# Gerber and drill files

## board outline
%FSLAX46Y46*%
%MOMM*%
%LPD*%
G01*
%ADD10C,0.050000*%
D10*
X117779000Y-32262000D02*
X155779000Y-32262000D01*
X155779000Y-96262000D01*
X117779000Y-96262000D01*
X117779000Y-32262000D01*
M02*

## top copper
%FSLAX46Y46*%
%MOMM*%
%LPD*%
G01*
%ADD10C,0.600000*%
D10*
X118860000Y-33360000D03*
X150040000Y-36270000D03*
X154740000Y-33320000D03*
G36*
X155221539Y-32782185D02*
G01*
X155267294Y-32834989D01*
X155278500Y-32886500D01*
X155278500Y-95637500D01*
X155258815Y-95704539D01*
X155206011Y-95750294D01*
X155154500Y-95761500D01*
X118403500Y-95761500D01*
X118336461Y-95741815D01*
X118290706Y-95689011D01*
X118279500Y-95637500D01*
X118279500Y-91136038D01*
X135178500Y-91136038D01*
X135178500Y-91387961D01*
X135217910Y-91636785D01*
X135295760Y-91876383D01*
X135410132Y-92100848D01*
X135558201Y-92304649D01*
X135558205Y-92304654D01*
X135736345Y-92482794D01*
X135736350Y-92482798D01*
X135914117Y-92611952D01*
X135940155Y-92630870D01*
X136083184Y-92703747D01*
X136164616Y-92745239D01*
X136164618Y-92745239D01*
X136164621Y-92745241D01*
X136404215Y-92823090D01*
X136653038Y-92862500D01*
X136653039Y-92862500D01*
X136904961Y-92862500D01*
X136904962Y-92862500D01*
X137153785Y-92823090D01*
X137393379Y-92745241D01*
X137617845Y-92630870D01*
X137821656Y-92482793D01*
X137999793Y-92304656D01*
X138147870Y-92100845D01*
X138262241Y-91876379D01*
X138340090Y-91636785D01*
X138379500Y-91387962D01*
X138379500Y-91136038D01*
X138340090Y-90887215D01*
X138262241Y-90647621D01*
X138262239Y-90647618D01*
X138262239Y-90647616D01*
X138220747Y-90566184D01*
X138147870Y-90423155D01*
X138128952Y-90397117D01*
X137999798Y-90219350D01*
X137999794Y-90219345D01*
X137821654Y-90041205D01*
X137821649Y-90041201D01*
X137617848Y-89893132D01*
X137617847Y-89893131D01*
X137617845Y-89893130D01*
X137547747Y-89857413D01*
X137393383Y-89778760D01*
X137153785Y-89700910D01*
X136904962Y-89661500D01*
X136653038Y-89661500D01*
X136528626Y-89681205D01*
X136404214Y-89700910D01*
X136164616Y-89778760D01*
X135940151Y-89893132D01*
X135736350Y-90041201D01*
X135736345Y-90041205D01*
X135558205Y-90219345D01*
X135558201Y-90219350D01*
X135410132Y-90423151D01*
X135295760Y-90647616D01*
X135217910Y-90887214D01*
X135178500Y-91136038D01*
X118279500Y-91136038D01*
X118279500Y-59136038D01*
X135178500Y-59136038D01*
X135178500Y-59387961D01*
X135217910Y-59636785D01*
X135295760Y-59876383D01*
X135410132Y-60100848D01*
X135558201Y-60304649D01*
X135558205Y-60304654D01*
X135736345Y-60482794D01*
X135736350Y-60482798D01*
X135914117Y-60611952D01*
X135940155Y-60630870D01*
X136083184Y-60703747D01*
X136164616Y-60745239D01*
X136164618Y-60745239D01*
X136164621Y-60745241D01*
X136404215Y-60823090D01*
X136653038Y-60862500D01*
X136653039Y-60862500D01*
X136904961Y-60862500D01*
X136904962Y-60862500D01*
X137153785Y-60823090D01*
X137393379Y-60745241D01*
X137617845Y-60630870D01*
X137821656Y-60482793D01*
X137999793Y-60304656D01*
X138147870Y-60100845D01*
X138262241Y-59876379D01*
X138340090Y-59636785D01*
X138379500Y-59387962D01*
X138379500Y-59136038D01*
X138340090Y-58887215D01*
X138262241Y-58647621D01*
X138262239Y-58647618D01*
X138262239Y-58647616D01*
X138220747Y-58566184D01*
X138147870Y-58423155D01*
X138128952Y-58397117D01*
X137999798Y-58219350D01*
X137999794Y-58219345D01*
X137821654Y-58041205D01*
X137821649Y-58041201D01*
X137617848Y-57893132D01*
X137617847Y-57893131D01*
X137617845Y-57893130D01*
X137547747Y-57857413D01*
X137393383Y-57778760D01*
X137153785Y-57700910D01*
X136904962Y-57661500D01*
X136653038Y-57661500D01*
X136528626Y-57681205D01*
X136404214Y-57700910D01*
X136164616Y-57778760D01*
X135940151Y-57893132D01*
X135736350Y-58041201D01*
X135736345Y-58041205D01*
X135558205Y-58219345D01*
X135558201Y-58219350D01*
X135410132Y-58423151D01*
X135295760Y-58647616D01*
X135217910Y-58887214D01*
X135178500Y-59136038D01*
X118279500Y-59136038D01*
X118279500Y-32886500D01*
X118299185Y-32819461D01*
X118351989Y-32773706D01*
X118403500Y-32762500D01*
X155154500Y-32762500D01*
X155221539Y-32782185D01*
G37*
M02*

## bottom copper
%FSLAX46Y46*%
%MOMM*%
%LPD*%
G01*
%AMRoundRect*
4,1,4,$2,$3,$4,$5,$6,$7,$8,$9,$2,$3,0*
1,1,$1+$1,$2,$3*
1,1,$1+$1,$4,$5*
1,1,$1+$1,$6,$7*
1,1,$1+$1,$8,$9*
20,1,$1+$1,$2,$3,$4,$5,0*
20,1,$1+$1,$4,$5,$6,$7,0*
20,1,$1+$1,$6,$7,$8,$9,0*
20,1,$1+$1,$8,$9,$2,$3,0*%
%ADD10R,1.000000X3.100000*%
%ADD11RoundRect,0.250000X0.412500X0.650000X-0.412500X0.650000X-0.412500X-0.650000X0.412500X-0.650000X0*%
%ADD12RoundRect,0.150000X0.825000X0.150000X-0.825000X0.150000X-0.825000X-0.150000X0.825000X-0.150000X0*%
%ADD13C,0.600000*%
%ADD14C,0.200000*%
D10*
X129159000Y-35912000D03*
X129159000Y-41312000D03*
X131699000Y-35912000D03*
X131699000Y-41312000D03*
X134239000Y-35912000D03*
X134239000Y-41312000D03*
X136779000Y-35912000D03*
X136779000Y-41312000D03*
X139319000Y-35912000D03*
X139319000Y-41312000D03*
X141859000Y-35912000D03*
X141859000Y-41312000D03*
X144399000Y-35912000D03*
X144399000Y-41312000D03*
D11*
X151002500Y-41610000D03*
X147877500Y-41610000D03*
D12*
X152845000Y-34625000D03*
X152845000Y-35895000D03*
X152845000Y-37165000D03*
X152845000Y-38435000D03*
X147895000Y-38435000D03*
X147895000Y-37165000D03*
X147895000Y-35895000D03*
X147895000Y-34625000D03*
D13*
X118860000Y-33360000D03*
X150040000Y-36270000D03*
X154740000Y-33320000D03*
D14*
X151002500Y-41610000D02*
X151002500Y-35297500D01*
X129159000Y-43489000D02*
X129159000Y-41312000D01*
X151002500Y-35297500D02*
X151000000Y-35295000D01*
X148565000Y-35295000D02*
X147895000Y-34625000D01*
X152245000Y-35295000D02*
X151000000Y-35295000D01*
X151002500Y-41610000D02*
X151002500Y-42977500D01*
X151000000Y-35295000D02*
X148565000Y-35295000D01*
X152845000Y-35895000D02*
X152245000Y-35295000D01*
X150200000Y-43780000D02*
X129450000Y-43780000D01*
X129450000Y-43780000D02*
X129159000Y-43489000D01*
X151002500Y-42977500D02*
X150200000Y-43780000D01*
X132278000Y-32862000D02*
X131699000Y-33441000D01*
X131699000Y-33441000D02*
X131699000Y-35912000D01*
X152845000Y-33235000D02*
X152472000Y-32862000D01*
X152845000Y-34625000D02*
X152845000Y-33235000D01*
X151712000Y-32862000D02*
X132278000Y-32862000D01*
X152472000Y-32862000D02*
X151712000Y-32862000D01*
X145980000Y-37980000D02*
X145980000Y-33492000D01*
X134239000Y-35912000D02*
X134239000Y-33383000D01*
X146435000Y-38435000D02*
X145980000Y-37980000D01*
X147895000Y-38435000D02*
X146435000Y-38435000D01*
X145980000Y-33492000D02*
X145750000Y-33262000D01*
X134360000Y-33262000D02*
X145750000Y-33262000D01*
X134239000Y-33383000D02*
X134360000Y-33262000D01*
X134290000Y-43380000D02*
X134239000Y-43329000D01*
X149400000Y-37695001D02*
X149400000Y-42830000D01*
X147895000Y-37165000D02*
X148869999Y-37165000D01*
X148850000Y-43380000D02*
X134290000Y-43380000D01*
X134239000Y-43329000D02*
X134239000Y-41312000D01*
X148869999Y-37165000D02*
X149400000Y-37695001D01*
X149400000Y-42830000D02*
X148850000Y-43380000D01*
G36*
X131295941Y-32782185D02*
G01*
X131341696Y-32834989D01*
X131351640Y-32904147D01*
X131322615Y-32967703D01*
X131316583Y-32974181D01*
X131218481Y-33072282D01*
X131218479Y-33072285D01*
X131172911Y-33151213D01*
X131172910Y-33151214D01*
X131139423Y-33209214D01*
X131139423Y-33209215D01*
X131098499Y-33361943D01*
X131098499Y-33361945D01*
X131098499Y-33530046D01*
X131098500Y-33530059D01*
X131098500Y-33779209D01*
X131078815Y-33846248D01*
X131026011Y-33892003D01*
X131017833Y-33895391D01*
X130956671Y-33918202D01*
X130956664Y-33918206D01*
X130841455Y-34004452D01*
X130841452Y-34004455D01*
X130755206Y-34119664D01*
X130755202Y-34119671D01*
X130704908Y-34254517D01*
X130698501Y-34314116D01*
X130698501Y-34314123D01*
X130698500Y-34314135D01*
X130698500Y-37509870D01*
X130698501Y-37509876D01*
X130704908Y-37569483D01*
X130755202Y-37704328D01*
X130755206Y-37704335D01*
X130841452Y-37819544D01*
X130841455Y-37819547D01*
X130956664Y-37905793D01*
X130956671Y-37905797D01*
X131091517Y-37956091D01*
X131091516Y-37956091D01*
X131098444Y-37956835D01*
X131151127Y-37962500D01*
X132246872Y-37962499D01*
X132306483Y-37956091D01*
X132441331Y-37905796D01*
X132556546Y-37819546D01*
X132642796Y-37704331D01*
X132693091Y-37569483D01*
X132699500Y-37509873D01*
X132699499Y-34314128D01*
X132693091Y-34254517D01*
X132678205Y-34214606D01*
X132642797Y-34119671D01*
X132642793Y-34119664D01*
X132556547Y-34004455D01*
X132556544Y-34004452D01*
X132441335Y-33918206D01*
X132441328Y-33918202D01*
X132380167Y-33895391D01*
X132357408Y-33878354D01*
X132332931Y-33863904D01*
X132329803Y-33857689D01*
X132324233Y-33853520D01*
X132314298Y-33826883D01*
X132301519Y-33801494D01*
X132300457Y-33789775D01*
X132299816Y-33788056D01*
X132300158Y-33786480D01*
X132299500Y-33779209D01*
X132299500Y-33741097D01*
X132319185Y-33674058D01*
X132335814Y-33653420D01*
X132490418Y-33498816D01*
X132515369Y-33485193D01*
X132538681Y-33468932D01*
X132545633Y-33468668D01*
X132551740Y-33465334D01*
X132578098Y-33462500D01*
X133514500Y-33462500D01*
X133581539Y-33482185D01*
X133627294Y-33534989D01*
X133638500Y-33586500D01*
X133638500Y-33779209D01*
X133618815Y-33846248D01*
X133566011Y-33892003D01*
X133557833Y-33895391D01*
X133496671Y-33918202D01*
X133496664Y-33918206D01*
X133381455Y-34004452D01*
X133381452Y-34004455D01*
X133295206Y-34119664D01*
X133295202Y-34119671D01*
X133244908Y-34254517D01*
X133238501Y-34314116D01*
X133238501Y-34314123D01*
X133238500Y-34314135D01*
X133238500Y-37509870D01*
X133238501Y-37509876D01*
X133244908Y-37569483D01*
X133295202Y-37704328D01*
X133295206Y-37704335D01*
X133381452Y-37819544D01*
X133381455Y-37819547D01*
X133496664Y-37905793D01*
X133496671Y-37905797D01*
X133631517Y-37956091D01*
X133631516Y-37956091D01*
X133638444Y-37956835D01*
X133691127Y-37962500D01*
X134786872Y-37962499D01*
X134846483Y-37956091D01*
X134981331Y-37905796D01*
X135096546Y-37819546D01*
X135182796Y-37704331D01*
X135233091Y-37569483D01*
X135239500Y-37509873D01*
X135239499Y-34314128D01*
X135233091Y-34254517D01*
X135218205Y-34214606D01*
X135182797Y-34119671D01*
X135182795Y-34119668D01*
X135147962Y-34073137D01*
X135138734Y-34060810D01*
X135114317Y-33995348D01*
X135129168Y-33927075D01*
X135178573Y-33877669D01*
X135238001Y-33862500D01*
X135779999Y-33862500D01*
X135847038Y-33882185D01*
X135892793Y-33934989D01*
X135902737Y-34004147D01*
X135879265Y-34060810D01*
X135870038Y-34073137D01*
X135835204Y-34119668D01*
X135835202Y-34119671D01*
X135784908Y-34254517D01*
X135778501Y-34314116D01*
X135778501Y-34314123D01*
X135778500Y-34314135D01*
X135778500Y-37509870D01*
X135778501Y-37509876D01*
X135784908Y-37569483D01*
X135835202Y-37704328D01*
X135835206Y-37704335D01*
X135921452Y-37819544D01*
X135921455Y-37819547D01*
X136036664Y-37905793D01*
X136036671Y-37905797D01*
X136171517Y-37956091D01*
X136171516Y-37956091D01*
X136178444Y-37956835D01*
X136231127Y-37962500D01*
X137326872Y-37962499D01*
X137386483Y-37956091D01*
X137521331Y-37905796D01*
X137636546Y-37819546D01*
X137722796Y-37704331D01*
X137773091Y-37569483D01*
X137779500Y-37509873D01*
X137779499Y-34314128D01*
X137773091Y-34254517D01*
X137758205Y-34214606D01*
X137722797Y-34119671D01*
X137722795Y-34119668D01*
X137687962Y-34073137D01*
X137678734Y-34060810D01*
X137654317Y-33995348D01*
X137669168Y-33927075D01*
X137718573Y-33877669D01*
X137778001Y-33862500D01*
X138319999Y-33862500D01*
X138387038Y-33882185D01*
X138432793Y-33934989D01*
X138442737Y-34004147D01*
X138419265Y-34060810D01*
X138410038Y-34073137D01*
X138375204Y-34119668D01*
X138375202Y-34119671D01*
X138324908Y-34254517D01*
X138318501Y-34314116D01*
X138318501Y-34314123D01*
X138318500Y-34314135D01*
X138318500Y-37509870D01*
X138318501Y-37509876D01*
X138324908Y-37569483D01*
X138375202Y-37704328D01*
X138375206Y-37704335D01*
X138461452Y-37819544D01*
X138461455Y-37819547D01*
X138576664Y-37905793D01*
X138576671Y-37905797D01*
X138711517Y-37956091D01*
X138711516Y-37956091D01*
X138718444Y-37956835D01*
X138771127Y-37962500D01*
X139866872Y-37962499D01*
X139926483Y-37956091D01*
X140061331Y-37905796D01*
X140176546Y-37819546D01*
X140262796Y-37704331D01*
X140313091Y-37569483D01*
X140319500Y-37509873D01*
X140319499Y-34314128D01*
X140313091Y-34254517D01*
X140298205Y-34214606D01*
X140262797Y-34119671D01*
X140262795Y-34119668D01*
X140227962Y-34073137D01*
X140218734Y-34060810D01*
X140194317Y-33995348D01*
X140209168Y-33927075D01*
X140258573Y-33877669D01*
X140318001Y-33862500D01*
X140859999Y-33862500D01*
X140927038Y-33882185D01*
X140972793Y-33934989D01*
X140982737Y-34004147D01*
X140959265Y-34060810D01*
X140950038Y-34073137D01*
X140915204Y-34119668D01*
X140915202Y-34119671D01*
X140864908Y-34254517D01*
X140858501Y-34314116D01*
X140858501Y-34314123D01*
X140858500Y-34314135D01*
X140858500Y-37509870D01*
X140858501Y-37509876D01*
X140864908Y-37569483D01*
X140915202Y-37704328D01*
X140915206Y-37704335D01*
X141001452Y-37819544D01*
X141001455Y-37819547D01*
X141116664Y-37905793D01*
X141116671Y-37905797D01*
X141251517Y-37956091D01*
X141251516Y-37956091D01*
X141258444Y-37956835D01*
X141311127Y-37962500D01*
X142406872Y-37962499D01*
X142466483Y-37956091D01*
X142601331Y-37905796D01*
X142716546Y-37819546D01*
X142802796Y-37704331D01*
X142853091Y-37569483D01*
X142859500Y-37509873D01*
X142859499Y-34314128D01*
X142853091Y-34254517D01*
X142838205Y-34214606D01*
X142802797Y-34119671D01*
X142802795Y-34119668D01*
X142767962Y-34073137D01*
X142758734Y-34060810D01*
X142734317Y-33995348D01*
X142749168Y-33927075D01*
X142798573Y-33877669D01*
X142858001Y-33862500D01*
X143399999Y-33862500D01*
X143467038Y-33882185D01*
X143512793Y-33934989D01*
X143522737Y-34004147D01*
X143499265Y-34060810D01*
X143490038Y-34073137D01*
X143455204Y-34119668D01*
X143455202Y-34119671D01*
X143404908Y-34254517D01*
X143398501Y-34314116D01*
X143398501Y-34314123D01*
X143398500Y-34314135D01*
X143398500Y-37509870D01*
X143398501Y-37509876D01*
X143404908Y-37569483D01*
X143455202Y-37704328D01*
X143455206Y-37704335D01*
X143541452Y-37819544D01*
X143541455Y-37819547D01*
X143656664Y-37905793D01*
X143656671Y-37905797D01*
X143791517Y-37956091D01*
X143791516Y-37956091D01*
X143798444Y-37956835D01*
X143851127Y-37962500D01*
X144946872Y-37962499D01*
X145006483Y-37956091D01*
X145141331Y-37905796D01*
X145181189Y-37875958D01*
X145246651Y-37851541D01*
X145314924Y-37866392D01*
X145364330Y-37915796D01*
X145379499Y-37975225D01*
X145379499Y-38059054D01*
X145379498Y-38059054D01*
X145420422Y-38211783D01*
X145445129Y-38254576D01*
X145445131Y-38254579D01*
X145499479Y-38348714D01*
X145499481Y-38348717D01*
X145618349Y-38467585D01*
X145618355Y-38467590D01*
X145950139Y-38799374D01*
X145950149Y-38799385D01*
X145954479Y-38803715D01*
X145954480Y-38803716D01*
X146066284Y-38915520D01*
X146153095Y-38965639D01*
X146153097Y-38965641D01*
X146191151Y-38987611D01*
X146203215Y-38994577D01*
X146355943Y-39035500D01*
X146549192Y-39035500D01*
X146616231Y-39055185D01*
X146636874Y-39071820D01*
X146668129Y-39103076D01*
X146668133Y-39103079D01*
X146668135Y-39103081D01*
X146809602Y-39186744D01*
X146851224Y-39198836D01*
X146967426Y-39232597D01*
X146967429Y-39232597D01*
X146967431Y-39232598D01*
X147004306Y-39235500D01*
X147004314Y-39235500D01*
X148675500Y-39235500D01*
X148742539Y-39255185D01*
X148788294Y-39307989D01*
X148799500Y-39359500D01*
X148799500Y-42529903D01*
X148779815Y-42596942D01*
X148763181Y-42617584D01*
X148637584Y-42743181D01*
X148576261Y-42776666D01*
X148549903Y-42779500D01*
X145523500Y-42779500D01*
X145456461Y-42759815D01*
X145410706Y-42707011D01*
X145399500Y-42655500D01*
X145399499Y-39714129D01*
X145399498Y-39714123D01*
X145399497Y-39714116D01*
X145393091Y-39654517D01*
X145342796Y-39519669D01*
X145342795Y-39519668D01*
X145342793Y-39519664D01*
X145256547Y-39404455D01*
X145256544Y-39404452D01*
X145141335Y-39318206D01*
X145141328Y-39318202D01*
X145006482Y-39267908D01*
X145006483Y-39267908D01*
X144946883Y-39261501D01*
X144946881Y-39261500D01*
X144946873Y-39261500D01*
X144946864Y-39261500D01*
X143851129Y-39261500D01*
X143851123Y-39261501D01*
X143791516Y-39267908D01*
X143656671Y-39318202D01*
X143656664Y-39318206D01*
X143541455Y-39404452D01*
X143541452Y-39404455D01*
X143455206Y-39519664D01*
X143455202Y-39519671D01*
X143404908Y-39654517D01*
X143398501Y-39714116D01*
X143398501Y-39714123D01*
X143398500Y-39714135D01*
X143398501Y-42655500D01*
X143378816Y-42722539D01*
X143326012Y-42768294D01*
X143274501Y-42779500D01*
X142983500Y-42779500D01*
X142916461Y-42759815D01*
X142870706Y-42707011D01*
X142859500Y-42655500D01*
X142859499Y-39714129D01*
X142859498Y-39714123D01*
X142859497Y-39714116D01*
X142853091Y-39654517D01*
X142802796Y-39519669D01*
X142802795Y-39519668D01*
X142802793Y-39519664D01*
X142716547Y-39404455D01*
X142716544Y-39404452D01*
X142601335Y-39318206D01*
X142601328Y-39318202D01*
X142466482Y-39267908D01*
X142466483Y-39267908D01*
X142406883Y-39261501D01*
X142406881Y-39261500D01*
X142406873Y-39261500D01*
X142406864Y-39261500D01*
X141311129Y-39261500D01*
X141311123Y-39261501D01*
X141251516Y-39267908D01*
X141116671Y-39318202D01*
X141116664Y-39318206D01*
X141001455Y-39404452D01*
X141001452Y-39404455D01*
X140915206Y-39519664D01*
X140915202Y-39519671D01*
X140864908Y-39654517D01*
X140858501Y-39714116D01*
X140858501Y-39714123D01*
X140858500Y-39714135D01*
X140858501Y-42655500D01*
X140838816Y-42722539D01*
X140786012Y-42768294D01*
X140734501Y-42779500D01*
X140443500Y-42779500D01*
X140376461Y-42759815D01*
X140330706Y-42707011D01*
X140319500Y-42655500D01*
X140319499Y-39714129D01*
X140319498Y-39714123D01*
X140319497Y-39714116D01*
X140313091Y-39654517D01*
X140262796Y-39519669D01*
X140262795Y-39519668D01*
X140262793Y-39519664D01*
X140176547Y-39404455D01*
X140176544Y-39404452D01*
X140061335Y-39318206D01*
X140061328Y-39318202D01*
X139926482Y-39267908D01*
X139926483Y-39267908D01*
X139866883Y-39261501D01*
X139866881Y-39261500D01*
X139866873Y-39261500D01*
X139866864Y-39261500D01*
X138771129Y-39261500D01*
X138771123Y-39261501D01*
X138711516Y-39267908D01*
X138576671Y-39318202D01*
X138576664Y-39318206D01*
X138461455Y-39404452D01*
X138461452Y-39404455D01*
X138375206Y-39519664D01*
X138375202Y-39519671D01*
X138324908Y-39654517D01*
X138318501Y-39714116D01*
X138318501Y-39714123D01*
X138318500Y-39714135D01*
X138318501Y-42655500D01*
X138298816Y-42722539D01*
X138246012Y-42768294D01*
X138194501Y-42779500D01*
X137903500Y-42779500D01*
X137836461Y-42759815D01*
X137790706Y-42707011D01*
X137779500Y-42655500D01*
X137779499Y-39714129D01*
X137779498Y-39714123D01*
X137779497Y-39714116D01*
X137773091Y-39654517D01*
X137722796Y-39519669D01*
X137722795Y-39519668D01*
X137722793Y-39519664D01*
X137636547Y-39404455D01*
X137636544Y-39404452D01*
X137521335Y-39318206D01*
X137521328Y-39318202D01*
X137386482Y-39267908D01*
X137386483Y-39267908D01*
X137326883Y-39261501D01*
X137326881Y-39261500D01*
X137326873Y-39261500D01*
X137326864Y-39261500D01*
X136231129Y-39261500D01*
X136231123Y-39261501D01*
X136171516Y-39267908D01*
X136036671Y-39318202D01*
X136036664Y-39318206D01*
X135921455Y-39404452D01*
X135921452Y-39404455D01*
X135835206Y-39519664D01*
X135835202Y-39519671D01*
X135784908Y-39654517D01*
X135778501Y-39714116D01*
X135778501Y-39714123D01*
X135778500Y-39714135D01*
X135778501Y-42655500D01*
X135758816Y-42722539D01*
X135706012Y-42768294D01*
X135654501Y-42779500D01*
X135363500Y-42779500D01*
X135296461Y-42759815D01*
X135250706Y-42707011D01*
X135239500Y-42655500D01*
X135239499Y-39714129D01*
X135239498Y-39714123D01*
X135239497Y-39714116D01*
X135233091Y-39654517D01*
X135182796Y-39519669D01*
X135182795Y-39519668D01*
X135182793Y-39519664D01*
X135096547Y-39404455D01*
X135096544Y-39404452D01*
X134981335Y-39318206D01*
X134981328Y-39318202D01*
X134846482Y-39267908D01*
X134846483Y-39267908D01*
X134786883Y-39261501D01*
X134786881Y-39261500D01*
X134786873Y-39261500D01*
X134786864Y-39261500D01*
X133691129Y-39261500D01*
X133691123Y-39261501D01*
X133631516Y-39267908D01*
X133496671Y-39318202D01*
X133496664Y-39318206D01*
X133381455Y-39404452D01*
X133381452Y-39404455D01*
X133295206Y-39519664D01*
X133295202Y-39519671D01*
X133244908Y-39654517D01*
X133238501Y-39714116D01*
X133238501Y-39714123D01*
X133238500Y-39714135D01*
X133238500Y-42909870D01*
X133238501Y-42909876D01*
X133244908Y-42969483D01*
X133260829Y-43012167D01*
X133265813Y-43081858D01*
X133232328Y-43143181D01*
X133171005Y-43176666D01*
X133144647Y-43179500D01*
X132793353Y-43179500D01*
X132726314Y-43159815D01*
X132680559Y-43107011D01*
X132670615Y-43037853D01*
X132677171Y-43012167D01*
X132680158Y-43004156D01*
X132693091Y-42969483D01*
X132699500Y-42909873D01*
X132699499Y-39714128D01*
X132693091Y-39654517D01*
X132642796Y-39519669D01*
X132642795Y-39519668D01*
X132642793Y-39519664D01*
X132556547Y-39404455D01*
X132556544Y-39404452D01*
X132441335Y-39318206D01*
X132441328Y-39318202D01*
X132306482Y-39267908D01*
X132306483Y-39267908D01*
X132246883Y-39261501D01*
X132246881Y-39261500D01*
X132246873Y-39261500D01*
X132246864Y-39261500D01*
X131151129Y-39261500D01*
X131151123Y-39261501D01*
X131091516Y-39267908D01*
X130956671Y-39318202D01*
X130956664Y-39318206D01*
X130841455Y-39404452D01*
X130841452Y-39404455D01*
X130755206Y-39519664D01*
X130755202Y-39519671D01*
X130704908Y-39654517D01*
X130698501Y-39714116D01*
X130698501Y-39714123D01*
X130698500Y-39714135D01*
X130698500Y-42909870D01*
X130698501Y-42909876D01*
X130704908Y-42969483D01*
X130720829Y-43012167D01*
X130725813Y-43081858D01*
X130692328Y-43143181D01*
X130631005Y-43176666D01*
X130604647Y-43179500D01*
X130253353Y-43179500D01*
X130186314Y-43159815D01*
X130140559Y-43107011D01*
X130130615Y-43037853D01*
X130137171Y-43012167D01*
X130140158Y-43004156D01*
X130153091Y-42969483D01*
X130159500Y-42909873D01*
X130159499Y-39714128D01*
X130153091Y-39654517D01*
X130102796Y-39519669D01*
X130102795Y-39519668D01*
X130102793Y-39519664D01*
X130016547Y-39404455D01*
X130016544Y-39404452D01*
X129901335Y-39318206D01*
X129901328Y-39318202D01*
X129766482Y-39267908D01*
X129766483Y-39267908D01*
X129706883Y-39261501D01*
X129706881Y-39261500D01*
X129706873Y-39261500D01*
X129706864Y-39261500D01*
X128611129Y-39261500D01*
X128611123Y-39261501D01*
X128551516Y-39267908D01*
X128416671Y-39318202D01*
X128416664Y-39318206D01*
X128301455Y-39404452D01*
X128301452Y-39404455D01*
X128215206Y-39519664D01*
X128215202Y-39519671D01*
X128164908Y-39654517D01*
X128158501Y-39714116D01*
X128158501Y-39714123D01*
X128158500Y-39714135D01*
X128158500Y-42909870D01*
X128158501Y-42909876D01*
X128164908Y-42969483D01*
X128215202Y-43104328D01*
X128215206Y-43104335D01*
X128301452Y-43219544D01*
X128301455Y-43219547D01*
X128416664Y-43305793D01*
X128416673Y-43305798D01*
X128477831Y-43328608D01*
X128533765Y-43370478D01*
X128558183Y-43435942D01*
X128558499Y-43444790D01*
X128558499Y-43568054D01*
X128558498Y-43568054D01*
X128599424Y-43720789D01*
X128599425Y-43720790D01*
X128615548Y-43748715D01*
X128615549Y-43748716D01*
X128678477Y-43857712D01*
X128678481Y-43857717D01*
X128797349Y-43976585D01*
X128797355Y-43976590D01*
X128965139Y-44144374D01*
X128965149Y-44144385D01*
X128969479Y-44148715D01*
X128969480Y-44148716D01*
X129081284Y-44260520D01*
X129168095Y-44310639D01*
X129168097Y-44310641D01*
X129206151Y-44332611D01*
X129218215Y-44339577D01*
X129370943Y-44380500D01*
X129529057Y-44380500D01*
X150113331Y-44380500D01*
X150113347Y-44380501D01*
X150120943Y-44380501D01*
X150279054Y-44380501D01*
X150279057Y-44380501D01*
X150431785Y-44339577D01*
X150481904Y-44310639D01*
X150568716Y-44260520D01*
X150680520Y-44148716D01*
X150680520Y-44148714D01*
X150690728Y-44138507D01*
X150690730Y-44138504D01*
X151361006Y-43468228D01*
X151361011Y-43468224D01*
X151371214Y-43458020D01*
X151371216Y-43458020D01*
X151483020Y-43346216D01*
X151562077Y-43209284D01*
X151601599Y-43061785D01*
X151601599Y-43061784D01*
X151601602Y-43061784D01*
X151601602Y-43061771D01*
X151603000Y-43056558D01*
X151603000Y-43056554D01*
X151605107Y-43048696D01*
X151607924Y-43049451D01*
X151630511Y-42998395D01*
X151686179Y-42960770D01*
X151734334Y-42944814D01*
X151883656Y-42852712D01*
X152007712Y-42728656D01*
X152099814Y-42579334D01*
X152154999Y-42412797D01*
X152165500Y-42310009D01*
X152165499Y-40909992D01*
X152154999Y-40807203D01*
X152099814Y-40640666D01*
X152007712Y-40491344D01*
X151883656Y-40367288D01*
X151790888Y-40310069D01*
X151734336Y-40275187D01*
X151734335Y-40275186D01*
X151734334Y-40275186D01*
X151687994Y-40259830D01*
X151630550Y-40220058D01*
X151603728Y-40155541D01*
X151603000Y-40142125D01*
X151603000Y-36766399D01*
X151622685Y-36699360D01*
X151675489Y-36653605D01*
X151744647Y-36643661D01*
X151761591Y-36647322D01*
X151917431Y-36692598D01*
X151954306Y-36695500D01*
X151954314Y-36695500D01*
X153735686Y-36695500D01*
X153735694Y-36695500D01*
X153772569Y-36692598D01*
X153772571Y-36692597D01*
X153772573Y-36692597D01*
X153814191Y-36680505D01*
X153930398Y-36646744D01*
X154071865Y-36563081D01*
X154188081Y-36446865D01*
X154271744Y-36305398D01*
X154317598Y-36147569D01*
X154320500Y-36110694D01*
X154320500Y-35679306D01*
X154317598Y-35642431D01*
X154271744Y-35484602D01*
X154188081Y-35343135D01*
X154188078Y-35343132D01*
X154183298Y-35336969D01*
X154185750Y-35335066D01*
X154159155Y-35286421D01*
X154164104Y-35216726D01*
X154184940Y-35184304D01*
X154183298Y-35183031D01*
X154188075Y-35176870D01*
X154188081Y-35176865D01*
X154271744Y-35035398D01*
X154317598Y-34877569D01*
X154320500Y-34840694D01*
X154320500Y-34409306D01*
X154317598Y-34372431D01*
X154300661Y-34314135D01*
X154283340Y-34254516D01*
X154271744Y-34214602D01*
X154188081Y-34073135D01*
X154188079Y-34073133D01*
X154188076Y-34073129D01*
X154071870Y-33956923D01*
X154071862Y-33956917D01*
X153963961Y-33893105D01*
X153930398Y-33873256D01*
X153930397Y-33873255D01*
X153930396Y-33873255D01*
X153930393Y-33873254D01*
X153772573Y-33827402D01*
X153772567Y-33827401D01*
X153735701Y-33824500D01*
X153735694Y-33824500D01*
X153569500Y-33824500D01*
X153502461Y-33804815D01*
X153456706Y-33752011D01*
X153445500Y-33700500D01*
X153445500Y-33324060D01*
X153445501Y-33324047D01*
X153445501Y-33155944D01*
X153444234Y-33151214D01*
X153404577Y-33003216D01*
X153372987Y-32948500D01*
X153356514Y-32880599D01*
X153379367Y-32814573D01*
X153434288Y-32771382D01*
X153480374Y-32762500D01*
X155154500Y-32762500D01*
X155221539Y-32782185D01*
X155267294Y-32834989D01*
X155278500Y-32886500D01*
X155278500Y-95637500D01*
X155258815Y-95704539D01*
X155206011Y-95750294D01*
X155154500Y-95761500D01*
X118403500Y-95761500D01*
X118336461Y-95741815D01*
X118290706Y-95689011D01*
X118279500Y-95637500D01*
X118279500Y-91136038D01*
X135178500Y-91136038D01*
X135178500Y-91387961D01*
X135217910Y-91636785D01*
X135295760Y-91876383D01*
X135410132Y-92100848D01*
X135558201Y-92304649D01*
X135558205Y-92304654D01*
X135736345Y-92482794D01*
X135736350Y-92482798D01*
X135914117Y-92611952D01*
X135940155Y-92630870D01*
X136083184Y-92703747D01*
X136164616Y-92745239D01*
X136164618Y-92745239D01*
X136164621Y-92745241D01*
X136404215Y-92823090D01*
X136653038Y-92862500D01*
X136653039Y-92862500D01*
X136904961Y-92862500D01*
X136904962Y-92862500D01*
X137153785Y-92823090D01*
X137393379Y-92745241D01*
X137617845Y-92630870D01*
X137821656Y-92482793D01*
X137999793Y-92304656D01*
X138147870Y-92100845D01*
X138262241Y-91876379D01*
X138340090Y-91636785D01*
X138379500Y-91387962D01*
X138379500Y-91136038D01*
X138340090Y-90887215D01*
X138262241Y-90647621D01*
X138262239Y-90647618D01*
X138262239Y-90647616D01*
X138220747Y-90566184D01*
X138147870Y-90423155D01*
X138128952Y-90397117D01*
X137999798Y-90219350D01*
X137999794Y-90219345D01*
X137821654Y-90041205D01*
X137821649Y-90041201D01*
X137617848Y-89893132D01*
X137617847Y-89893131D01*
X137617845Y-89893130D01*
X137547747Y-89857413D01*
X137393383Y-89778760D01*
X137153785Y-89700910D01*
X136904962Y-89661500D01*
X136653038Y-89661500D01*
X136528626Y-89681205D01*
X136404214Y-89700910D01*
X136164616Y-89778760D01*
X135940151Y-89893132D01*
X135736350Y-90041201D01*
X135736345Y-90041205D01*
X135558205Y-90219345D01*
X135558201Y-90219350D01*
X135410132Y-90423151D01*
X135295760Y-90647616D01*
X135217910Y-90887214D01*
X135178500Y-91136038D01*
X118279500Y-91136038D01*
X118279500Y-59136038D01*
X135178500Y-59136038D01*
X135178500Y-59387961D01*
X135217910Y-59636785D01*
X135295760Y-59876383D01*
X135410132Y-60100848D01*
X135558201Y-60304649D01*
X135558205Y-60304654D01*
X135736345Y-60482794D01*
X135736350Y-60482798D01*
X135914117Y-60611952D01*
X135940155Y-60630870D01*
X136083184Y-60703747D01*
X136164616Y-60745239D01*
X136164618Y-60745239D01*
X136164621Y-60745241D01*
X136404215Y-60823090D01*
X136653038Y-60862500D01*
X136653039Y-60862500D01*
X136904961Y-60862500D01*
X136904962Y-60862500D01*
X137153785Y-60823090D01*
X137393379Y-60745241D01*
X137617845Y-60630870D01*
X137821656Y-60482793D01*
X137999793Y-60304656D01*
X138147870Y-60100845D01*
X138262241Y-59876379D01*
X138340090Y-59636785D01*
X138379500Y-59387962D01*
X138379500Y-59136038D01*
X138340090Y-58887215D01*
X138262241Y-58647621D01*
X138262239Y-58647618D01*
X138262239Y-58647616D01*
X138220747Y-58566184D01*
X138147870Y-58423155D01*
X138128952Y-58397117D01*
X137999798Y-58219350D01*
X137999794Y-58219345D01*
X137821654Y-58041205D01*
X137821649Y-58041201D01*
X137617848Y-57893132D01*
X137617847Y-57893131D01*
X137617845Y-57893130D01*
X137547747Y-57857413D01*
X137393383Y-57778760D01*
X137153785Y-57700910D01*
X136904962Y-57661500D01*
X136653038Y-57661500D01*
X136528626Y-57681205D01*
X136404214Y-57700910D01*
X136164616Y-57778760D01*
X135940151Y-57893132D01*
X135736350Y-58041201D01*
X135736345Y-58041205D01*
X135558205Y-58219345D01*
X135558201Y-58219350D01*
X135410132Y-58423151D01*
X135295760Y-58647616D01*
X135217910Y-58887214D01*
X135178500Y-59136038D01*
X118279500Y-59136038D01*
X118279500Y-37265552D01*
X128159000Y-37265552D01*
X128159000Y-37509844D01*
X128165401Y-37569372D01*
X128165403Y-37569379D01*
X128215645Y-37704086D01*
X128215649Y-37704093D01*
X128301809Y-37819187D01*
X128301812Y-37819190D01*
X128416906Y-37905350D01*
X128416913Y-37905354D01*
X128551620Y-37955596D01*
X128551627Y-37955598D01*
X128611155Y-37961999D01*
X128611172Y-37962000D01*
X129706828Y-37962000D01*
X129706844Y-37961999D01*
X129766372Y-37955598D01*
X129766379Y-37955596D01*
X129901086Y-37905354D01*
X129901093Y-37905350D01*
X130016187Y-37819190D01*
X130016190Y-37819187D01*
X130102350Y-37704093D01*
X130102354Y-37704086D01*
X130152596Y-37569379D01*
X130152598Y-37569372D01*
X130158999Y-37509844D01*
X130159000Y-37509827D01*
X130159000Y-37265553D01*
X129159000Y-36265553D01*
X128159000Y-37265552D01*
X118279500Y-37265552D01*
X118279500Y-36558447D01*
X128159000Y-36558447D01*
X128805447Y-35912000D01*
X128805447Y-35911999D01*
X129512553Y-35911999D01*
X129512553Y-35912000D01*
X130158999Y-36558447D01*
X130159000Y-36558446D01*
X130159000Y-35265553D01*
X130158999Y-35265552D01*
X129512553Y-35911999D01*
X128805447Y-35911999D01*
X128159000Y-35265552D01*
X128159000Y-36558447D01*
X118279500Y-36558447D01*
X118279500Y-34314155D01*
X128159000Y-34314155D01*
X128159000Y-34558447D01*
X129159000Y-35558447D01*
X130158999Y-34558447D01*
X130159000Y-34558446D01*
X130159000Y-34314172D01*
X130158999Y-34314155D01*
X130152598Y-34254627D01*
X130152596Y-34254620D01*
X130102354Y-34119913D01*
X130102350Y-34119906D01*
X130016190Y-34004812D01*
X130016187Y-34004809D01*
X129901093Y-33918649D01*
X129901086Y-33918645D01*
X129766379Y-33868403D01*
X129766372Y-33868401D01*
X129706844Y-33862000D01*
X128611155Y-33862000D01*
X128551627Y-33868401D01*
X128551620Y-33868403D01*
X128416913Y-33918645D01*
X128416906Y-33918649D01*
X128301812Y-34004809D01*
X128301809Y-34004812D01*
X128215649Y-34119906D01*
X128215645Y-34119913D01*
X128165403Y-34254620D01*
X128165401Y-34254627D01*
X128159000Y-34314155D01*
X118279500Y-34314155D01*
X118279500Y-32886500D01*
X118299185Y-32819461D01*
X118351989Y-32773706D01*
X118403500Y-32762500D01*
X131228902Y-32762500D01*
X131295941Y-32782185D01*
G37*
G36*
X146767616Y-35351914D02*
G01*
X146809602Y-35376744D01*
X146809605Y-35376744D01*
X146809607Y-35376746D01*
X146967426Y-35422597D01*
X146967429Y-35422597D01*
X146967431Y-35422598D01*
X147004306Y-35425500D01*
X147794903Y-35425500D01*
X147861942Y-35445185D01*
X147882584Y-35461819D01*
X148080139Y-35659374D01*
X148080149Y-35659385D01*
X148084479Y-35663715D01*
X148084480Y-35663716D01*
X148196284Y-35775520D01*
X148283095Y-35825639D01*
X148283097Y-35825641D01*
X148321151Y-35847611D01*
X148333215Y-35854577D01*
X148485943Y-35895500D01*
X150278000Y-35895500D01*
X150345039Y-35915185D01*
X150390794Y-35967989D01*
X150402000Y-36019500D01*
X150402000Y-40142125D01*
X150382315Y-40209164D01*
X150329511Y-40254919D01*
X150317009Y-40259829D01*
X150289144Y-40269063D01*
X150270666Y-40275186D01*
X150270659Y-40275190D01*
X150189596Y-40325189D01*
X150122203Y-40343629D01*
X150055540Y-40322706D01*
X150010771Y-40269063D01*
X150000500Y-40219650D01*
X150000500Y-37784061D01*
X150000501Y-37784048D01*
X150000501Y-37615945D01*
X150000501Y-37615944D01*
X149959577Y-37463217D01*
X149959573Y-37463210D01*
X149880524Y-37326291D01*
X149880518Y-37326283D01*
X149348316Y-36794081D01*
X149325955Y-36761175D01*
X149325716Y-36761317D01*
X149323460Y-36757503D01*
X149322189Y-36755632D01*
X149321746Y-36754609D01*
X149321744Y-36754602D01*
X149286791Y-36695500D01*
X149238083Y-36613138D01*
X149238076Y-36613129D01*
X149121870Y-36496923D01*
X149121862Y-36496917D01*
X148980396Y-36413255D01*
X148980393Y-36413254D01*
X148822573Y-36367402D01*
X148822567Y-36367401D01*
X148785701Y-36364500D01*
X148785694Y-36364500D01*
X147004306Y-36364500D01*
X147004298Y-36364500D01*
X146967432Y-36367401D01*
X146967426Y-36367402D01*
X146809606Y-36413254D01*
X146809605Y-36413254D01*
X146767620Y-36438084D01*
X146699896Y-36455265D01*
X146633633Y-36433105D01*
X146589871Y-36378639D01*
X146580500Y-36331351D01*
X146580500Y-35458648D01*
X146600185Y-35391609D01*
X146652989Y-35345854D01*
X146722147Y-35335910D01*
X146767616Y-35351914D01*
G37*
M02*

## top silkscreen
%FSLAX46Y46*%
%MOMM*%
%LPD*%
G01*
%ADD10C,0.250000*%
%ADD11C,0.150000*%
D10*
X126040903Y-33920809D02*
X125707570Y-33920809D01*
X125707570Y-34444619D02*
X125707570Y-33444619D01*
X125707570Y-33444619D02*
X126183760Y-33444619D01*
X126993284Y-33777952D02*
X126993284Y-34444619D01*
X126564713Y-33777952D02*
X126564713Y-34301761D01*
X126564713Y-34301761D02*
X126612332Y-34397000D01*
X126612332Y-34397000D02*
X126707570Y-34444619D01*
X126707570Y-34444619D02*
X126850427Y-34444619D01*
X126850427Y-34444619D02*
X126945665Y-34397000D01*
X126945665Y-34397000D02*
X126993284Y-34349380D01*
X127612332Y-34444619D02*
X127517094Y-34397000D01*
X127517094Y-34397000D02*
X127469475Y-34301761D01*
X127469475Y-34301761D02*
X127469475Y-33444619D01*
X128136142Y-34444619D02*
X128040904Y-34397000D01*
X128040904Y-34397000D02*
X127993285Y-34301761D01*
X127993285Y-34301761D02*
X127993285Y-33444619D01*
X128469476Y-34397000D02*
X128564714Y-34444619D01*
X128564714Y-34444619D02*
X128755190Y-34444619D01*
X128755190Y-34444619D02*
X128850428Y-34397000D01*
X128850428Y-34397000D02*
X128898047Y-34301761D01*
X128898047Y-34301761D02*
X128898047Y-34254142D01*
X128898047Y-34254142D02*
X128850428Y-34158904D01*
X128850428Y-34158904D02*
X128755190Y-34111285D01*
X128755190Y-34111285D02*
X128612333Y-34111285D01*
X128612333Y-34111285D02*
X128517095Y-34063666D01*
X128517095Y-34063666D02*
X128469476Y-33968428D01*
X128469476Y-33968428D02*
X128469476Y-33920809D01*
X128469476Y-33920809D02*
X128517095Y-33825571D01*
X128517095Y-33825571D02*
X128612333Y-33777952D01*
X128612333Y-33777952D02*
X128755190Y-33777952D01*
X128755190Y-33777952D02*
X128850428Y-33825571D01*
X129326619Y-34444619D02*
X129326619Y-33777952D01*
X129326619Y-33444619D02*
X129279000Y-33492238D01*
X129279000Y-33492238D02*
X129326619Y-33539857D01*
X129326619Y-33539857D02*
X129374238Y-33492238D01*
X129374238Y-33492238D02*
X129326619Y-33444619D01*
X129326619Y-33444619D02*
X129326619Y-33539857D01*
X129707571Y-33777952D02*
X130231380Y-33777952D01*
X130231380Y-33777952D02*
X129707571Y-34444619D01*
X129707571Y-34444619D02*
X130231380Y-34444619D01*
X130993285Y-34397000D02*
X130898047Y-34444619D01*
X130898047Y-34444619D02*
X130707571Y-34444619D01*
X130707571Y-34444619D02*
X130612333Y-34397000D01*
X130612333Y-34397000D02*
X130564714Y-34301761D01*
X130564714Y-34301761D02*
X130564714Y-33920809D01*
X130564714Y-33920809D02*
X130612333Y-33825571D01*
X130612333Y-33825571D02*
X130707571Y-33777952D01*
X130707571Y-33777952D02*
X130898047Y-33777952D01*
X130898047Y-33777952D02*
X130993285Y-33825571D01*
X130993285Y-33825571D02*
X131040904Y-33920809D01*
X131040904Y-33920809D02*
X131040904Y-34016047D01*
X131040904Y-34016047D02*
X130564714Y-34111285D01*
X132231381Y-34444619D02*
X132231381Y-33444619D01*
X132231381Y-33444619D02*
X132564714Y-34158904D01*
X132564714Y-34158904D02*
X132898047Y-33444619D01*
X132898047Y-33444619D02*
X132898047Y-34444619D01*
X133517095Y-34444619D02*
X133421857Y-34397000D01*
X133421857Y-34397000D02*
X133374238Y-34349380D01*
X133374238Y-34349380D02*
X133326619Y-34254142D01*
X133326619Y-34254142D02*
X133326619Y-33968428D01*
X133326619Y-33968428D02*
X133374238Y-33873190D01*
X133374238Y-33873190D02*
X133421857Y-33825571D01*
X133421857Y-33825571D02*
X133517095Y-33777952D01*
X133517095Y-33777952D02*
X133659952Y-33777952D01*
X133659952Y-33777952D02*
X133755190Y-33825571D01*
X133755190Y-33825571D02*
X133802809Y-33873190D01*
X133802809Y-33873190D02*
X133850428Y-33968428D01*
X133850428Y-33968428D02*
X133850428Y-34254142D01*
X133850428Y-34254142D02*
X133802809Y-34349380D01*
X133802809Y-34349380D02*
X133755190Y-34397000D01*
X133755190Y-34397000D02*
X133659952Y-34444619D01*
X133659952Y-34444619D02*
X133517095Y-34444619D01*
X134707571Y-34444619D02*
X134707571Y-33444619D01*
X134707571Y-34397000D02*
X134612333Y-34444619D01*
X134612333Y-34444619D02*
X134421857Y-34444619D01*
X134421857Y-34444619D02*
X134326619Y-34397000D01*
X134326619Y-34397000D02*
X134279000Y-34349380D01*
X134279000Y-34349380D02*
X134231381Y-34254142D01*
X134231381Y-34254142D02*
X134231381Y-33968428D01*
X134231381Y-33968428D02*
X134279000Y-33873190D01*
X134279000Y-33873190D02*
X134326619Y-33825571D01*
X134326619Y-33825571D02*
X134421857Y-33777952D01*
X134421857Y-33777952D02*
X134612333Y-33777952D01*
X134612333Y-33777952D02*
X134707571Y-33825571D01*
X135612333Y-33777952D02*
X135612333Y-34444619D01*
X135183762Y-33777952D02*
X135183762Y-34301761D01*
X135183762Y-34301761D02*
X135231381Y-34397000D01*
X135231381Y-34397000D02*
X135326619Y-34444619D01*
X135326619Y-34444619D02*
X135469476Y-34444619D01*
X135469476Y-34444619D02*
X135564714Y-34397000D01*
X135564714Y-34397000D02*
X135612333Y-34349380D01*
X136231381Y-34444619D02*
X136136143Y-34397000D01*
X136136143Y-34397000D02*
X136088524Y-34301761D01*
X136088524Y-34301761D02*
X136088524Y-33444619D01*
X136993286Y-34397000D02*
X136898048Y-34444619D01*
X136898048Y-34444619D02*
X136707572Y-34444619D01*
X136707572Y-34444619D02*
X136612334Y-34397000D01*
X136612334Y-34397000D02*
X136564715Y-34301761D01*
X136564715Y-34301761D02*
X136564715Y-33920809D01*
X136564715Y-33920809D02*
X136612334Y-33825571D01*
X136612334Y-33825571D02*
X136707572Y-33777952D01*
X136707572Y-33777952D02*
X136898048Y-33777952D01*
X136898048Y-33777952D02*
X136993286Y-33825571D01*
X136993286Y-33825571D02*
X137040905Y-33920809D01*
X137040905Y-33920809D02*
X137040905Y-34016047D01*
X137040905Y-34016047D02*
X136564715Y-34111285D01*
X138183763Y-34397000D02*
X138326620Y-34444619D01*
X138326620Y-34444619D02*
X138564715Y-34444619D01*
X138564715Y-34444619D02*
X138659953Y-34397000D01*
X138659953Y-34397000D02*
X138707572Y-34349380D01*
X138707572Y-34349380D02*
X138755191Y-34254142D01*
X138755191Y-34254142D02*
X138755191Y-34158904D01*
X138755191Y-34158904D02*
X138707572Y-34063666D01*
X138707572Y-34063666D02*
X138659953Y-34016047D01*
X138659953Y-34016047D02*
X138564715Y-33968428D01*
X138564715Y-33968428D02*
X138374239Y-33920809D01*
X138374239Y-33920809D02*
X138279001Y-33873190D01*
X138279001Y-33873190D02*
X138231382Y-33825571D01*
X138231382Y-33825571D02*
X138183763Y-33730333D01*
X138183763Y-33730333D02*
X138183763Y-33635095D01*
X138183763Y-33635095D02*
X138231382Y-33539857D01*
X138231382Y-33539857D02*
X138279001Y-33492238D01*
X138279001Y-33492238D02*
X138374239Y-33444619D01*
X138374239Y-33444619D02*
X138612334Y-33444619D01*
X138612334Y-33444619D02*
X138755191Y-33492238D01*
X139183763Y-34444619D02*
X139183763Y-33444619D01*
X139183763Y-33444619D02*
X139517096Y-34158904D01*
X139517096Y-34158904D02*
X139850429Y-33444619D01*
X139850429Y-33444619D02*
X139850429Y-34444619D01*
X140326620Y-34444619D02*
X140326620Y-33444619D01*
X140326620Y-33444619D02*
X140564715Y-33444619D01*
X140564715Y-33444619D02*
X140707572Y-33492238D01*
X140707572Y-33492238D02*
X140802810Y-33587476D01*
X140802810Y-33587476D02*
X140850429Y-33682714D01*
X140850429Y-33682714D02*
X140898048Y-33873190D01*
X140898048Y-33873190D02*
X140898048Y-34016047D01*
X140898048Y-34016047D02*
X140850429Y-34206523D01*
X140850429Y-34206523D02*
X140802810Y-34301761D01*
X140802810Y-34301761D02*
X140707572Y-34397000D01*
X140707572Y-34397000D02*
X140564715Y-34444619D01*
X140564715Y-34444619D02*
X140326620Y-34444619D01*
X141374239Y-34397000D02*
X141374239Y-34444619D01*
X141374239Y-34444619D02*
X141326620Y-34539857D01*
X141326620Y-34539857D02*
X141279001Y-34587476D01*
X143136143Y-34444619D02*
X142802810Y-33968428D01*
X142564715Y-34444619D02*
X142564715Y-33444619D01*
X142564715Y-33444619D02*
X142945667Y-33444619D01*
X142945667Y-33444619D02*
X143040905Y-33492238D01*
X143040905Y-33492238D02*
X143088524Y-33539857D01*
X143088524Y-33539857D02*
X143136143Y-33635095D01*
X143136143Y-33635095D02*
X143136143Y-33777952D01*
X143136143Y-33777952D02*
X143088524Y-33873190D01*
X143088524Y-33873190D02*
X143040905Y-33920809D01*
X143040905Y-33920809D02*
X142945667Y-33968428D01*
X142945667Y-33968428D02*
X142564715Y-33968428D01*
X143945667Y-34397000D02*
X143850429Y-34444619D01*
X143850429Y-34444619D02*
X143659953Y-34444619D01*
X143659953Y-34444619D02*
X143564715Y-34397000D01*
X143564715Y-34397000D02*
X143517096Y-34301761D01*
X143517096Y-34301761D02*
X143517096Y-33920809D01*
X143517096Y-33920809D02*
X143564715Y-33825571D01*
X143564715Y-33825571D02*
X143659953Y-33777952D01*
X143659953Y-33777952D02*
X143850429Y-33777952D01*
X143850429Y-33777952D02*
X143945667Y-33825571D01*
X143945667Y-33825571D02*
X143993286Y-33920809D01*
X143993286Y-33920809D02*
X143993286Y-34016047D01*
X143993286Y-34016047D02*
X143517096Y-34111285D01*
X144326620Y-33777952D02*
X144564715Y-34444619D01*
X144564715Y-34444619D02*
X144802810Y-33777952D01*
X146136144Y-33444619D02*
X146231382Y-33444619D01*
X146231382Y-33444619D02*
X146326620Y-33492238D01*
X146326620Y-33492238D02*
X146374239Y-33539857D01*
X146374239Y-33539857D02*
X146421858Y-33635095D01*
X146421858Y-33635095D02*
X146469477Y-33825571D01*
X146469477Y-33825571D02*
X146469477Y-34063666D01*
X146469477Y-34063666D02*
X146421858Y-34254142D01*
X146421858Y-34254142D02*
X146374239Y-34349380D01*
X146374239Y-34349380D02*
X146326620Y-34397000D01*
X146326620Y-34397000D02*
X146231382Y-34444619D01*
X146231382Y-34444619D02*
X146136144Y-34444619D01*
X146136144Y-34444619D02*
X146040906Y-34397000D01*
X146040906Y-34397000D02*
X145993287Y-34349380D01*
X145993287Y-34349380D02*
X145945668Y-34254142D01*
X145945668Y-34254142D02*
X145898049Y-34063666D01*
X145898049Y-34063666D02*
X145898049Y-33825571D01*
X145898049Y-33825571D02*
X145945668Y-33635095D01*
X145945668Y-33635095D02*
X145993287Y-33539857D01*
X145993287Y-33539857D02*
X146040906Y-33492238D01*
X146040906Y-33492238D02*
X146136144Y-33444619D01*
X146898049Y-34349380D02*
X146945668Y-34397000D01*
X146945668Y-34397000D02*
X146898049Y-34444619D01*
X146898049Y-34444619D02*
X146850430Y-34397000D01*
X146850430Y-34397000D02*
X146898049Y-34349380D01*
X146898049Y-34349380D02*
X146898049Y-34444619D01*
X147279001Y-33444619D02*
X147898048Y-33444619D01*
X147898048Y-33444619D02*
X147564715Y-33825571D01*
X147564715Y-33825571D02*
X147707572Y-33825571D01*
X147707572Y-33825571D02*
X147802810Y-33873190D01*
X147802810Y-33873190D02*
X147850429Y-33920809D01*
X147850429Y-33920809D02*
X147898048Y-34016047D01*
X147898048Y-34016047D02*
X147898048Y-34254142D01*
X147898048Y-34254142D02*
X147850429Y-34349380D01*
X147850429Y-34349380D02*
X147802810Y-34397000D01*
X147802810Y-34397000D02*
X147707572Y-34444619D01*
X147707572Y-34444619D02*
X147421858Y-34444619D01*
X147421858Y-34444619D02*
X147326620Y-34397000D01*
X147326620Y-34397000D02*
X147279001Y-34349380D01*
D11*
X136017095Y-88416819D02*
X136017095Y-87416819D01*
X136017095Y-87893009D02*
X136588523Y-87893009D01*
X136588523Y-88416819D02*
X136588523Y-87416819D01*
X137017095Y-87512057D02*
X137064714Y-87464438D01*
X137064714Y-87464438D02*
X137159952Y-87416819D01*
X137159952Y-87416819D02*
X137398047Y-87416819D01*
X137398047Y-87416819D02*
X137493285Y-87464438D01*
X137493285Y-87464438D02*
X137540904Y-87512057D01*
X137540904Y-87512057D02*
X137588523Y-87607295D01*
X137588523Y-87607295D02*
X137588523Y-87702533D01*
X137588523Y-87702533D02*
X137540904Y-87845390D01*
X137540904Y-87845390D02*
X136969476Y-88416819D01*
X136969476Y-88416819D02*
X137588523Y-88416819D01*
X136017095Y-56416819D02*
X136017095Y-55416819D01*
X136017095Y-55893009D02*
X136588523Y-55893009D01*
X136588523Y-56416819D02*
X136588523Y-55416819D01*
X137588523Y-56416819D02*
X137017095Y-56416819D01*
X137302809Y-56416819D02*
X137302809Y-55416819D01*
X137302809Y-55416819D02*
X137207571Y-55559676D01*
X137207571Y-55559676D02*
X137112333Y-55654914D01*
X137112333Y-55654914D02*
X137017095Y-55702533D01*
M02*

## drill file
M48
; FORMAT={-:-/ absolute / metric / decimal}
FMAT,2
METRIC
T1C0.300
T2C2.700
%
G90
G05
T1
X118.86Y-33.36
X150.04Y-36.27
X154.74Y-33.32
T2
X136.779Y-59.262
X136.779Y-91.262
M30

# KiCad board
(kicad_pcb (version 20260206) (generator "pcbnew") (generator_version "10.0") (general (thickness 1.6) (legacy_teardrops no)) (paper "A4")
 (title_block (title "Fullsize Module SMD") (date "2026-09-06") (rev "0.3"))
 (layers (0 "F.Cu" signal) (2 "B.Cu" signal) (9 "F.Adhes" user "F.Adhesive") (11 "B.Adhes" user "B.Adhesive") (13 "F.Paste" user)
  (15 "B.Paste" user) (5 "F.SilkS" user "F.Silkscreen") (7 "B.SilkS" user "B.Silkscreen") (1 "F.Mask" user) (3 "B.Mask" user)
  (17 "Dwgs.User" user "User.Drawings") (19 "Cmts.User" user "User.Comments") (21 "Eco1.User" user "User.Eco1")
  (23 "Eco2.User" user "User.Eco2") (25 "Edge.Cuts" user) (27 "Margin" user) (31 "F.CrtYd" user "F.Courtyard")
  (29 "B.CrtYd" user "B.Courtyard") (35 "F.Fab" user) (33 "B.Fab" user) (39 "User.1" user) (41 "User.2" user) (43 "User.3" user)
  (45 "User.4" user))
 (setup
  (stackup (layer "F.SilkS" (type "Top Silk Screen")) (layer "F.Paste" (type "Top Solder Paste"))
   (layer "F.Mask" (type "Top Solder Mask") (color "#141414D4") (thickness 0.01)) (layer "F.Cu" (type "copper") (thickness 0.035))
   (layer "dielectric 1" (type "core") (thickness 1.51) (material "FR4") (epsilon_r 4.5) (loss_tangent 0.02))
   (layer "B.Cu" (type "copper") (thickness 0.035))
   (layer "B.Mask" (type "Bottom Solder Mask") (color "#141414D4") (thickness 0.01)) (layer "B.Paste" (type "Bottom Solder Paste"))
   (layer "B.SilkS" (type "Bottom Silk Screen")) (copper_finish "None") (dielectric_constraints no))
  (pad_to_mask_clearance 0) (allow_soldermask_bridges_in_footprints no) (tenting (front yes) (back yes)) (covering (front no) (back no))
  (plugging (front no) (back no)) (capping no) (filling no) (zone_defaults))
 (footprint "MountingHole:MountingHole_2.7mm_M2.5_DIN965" (layer "F.Cu") (at 136.779 91.262)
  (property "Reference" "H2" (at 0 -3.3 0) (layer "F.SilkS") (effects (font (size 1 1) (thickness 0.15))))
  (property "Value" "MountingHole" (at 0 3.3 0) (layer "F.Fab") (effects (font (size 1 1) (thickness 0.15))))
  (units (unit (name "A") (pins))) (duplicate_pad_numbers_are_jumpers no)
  (pad "" np_thru_hole circle (at 0 0) (size 2.7 2.7) (drill 2.7) (layers "*.Cu" "*.Mask")))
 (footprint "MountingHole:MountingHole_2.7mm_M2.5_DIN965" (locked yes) (layer "F.Cu") (at 136.779 59.262)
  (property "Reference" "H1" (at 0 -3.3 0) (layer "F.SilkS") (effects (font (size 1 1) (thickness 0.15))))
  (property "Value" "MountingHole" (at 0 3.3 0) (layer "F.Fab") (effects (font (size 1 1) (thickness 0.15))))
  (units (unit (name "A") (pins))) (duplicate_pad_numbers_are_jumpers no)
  (pad "" np_thru_hole circle (at 0 0) (size 2.7 2.7) (drill 2.7) (layers "*.Cu" "*.Mask")))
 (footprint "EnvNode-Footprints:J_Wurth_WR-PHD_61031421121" (layer "B.Cu") (at 136.779 38.612 -90)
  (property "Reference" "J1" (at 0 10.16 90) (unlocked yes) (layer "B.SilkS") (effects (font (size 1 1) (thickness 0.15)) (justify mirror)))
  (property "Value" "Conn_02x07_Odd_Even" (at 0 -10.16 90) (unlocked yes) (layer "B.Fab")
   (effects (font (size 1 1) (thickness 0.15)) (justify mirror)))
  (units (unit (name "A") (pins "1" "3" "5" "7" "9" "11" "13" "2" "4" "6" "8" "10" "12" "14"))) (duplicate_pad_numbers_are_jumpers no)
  (pad "1" smd rect (at -2.7 7.62) (size 1 3.1) (layers "B.Cu" "B.Mask" "B.Paste") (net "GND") (thermal_bridge_angle 45))
  (pad "2" smd rect (at 2.7 7.62) (size 1 3.1) (layers "B.Cu" "B.Mask" "B.Paste") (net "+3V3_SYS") (thermal_bridge_angle 45))
  (pad "3" smd rect (at -2.7 5.08) (size 1 3.1) (layers "B.Cu" "B.Mask" "B.Paste") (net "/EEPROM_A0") (thermal_bridge_angle 45))
  (pad "4" smd rect (at 2.7 5.08) (size 1 3.1) (layers "B.Cu" "B.Mask" "B.Paste") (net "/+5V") (thermal_bridge_angle 45))
  (pad "5" smd rect (at -2.7 2.54) (size 1 3.1) (layers "B.Cu" "B.Mask" "B.Paste") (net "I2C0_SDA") (thermal_bridge_angle 45))
  (pad "6" smd rect (at 2.7 2.54) (size 1 3.1) (layers "B.Cu" "B.Mask" "B.Paste") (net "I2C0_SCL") (thermal_bridge_angle 45))
  (pad "7" smd rect (at -2.7 0) (size 1 3.1) (layers "B.Cu" "B.Mask" "B.Paste") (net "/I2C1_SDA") (thermal_bridge_angle 45))
  (pad "8" smd rect (at 2.7 0) (size 1 3.1) (layers "B.Cu" "B.Mask" "B.Paste") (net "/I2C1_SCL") (thermal_bridge_angle 45))
  (pad "9" smd rect (at -2.7 -2.54) (size 1 3.1) (layers "B.Cu" "B.Mask" "B.Paste") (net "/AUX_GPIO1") (thermal_bridge_angle 45))
  (pad "10" smd rect (at 2.7 -2.54) (size 1 3.1) (layers "B.Cu" "B.Mask" "B.Paste") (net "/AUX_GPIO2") (thermal_bridge_angle 45))
  (pad "11" smd rect (at -2.7 -5.08) (size 1 3.1) (layers "B.Cu" "B.Mask" "B.Paste") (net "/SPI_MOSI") (thermal_bridge_angle 45))
  (pad "12" smd rect (at 2.7 -5.08) (size 1 3.1) (layers "B.Cu" "B.Mask" "B.Paste") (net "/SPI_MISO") (thermal_bridge_angle 45))
  (pad "13" smd rect (at -2.7 -7.62) (size 1 3.1) (layers "B.Cu" "B.Mask" "B.Paste") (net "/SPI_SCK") (thermal_bridge_angle 45))
  (pad "14" smd rect (at 2.7 -7.62) (size 1 3.1) (layers "B.Cu" "B.Mask" "B.Paste") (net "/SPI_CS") (thermal_bridge_angle 45)))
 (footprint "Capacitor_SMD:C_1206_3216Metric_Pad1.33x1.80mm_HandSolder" (layer "B.Cu") (at 149.44 41.61 180)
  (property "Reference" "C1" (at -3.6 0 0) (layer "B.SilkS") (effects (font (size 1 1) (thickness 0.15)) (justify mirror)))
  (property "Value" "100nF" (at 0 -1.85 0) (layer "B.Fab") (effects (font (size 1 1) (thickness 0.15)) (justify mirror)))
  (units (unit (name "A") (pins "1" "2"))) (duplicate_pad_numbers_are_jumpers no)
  (pad "1" smd roundrect (at -1.5625 0 180) (size 1.325 1.8) (layers "B.Cu" "B.Mask" "B.Paste") (roundrect_rratio 0.188679) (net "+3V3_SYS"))
  (pad "2" smd roundrect (at 1.5625 0 180) (size 1.325 1.8) (layers "B.Cu" "B.Mask" "B.Paste") (roundrect_rratio 0.188679) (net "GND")
   (zone_connect 2)))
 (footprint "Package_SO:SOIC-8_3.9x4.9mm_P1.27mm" (layer "B.Cu") (at 150.37 36.53 180)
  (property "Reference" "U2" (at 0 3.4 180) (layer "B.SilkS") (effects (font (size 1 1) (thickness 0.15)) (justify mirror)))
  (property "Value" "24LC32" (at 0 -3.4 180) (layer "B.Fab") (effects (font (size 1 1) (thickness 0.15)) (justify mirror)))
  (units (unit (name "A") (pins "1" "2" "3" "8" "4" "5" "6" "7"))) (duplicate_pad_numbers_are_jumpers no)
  (pad "1" smd roundrect (at -2.475 1.905 180) (size 1.95 0.6) (layers "B.Cu" "B.Mask" "B.Paste") (roundrect_rratio 0.25) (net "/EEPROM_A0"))
  (pad "2" smd roundrect (at -2.475 0.635 180) (size 1.95 0.6) (layers "B.Cu" "B.Mask" "B.Paste") (roundrect_rratio 0.25) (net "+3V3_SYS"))
  (pad "3" smd roundrect (at -2.475 -0.635 180) (size 1.95 0.6) (layers "B.Cu" "B.Mask" "B.Paste") (roundrect_rratio 0.25) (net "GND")
   (zone_connect 2))
  (pad "4" smd roundrect (at -2.475 -1.905 180) (size 1.95 0.6) (layers "B.Cu" "B.Mask" "B.Paste") (roundrect_rratio 0.25) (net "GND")
   (zone_connect 2))
  (pad "5" smd roundrect (at 2.475 -1.905 180) (size 1.95 0.6) (layers "B.Cu" "B.Mask" "B.Paste") (roundrect_rratio 0.25) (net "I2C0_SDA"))
  (pad "6" smd roundrect (at 2.475 -0.635 180) (size 1.95 0.6) (layers "B.Cu" "B.Mask" "B.Paste") (roundrect_rratio 0.25) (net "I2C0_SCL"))
  (pad "7" smd roundrect (at 2.475 0.635 180) (size 1.95 0.6) (layers "B.Cu" "B.Mask" "B.Paste") (roundrect_rratio 0.25) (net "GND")
   (zone_connect 2))
  (pad "8" smd roundrect (at 2.475 1.905 180) (size 1.95 0.6) (layers "B.Cu" "B.Mask" "B.Paste") (roundrect_rratio 0.25) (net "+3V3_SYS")))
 (gr_rect (start 117.779 32.262) (end 155.779 96.262) (stroke (width 0.05) (type solid)) (fill no) (layer "Edge.Cuts"))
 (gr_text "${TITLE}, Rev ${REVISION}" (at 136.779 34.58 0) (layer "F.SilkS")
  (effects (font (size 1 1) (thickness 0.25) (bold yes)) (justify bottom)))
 (via (at 118.86 33.36) (size 0.6) (drill 0.3) (layers "F.Cu" "B.Cu") (free yes) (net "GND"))
 (via (at 150.04 36.27) (size 0.6) (drill 0.3) (layers "F.Cu" "B.Cu") (free yes) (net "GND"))
 (via (at 154.74 33.32) (size 0.6) (drill 0.3) (layers "F.Cu" "B.Cu") (free yes) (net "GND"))
 (segment (start 151.0025 41.61) (end 151.0025 35.2975) (width 0.2) (layer "B.Cu") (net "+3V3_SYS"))
 (segment (start 129.159 43.489) (end 129.159 41.312) (width 0.2) (layer "B.Cu") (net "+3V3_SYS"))
 (segment (start 151.0025 35.2975) (end 151 35.295) (width 0.2) (layer "B.Cu") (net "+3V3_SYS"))
 (segment (start 148.565 35.295) (end 147.895 34.625) (width 0.2) (layer "B.Cu") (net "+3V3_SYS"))
 (segment (start 152.245 35.295) (end 151 35.295) (width 0.2) (layer "B.Cu") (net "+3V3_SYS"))
 (segment (start 151.0025 41.61) (end 151.0025 42.9775) (width 0.2) (layer "B.Cu") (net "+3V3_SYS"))
 (segment (start 151 35.295) (end 148.565 35.295) (width 0.2) (layer "B.Cu") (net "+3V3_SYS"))
 (segment (start 152.845 35.895) (end 152.245 35.295) (width 0.2) (layer "B.Cu") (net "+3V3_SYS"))
 (segment (start 150.2 43.78) (end 129.45 43.78) (width 0.2) (layer "B.Cu") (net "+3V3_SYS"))
 (segment (start 129.45 43.78) (end 129.159 43.489) (width 0.2) (layer "B.Cu") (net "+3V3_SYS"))
 (segment (start 151.0025 42.9775) (end 150.2 43.78) (width 0.2) (layer "B.Cu") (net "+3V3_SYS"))
 (segment (start 132.278 32.862) (end 131.699 33.441) (width 0.2) (layer "B.Cu") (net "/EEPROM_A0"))
 (segment (start 131.699 33.441) (end 131.699 35.912) (width 0.2) (layer "B.Cu") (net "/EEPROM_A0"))
 (segment (start 152.845 33.235) (end 152.472 32.862) (width 0.2) (layer "B.Cu") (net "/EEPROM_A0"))
 (segment (start 152.845 34.625) (end 152.845 33.235) (width 0.2) (layer "B.Cu") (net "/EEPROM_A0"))
 (segment (start 151.712 32.862) (end 132.278 32.862) (width 0.2) (layer "B.Cu") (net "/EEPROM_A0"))
 (segment (start 152.472 32.862) (end 151.712 32.862) (width 0.2) (layer "B.Cu") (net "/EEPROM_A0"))
 (segment (start 145.98 37.98) (end 145.98 33.492) (width 0.2) (layer "B.Cu") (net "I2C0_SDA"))
 (segment (start 134.239 35.912) (end 134.239 33.383) (width 0.2) (layer "B.Cu") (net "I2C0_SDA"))
 (segment (start 146.435 38.435) (end 145.98 37.98) (width 0.2) (layer "B.Cu") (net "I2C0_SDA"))
 (segment (start 147.895 38.435) (end 146.435 38.435) (width 0.2) (layer "B.Cu") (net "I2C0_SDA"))
 (segment (start 145.98 33.492) (end 145.75 33.262) (width 0.2) (layer "B.Cu") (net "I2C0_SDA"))
 (segment (start 134.36 33.262) (end 145.75 33.262) (width 0.2) (layer "B.Cu") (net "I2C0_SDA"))
 (segment (start 134.239 33.383) (end 134.36 33.262) (width 0.2) (layer "B.Cu") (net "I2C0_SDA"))
 (segment (start 134.29 43.38) (end 134.239 43.329) (width 0.2) (layer "B.Cu") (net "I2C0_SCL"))
 (segment (start 149.4 37.695001) (end 149.4 42.83) (width 0.2) (layer "B.Cu") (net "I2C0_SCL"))
 (segment (start 147.895 37.165) (end 148.869999 37.165) (width 0.2) (layer "B.Cu") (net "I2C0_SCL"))
 (segment (start 148.85 43.38) (end 134.29 43.38) (width 0.2) (layer "B.Cu") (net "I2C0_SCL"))
 (segment (start 134.239 43.329) (end 134.239 41.312) (width 0.2) (layer "B.Cu") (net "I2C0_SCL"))
 (segment (start 148.869999 37.165) (end 149.4 37.695001) (width 0.2) (layer "B.Cu") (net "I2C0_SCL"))
 (segment (start 149.4 42.83) (end 148.85 43.38) (width 0.2) (layer "B.Cu") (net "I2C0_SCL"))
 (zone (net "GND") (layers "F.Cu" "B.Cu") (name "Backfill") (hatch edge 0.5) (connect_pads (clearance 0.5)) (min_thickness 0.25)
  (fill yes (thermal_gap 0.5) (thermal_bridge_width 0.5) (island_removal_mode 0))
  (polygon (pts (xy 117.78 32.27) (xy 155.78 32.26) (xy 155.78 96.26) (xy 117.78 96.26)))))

